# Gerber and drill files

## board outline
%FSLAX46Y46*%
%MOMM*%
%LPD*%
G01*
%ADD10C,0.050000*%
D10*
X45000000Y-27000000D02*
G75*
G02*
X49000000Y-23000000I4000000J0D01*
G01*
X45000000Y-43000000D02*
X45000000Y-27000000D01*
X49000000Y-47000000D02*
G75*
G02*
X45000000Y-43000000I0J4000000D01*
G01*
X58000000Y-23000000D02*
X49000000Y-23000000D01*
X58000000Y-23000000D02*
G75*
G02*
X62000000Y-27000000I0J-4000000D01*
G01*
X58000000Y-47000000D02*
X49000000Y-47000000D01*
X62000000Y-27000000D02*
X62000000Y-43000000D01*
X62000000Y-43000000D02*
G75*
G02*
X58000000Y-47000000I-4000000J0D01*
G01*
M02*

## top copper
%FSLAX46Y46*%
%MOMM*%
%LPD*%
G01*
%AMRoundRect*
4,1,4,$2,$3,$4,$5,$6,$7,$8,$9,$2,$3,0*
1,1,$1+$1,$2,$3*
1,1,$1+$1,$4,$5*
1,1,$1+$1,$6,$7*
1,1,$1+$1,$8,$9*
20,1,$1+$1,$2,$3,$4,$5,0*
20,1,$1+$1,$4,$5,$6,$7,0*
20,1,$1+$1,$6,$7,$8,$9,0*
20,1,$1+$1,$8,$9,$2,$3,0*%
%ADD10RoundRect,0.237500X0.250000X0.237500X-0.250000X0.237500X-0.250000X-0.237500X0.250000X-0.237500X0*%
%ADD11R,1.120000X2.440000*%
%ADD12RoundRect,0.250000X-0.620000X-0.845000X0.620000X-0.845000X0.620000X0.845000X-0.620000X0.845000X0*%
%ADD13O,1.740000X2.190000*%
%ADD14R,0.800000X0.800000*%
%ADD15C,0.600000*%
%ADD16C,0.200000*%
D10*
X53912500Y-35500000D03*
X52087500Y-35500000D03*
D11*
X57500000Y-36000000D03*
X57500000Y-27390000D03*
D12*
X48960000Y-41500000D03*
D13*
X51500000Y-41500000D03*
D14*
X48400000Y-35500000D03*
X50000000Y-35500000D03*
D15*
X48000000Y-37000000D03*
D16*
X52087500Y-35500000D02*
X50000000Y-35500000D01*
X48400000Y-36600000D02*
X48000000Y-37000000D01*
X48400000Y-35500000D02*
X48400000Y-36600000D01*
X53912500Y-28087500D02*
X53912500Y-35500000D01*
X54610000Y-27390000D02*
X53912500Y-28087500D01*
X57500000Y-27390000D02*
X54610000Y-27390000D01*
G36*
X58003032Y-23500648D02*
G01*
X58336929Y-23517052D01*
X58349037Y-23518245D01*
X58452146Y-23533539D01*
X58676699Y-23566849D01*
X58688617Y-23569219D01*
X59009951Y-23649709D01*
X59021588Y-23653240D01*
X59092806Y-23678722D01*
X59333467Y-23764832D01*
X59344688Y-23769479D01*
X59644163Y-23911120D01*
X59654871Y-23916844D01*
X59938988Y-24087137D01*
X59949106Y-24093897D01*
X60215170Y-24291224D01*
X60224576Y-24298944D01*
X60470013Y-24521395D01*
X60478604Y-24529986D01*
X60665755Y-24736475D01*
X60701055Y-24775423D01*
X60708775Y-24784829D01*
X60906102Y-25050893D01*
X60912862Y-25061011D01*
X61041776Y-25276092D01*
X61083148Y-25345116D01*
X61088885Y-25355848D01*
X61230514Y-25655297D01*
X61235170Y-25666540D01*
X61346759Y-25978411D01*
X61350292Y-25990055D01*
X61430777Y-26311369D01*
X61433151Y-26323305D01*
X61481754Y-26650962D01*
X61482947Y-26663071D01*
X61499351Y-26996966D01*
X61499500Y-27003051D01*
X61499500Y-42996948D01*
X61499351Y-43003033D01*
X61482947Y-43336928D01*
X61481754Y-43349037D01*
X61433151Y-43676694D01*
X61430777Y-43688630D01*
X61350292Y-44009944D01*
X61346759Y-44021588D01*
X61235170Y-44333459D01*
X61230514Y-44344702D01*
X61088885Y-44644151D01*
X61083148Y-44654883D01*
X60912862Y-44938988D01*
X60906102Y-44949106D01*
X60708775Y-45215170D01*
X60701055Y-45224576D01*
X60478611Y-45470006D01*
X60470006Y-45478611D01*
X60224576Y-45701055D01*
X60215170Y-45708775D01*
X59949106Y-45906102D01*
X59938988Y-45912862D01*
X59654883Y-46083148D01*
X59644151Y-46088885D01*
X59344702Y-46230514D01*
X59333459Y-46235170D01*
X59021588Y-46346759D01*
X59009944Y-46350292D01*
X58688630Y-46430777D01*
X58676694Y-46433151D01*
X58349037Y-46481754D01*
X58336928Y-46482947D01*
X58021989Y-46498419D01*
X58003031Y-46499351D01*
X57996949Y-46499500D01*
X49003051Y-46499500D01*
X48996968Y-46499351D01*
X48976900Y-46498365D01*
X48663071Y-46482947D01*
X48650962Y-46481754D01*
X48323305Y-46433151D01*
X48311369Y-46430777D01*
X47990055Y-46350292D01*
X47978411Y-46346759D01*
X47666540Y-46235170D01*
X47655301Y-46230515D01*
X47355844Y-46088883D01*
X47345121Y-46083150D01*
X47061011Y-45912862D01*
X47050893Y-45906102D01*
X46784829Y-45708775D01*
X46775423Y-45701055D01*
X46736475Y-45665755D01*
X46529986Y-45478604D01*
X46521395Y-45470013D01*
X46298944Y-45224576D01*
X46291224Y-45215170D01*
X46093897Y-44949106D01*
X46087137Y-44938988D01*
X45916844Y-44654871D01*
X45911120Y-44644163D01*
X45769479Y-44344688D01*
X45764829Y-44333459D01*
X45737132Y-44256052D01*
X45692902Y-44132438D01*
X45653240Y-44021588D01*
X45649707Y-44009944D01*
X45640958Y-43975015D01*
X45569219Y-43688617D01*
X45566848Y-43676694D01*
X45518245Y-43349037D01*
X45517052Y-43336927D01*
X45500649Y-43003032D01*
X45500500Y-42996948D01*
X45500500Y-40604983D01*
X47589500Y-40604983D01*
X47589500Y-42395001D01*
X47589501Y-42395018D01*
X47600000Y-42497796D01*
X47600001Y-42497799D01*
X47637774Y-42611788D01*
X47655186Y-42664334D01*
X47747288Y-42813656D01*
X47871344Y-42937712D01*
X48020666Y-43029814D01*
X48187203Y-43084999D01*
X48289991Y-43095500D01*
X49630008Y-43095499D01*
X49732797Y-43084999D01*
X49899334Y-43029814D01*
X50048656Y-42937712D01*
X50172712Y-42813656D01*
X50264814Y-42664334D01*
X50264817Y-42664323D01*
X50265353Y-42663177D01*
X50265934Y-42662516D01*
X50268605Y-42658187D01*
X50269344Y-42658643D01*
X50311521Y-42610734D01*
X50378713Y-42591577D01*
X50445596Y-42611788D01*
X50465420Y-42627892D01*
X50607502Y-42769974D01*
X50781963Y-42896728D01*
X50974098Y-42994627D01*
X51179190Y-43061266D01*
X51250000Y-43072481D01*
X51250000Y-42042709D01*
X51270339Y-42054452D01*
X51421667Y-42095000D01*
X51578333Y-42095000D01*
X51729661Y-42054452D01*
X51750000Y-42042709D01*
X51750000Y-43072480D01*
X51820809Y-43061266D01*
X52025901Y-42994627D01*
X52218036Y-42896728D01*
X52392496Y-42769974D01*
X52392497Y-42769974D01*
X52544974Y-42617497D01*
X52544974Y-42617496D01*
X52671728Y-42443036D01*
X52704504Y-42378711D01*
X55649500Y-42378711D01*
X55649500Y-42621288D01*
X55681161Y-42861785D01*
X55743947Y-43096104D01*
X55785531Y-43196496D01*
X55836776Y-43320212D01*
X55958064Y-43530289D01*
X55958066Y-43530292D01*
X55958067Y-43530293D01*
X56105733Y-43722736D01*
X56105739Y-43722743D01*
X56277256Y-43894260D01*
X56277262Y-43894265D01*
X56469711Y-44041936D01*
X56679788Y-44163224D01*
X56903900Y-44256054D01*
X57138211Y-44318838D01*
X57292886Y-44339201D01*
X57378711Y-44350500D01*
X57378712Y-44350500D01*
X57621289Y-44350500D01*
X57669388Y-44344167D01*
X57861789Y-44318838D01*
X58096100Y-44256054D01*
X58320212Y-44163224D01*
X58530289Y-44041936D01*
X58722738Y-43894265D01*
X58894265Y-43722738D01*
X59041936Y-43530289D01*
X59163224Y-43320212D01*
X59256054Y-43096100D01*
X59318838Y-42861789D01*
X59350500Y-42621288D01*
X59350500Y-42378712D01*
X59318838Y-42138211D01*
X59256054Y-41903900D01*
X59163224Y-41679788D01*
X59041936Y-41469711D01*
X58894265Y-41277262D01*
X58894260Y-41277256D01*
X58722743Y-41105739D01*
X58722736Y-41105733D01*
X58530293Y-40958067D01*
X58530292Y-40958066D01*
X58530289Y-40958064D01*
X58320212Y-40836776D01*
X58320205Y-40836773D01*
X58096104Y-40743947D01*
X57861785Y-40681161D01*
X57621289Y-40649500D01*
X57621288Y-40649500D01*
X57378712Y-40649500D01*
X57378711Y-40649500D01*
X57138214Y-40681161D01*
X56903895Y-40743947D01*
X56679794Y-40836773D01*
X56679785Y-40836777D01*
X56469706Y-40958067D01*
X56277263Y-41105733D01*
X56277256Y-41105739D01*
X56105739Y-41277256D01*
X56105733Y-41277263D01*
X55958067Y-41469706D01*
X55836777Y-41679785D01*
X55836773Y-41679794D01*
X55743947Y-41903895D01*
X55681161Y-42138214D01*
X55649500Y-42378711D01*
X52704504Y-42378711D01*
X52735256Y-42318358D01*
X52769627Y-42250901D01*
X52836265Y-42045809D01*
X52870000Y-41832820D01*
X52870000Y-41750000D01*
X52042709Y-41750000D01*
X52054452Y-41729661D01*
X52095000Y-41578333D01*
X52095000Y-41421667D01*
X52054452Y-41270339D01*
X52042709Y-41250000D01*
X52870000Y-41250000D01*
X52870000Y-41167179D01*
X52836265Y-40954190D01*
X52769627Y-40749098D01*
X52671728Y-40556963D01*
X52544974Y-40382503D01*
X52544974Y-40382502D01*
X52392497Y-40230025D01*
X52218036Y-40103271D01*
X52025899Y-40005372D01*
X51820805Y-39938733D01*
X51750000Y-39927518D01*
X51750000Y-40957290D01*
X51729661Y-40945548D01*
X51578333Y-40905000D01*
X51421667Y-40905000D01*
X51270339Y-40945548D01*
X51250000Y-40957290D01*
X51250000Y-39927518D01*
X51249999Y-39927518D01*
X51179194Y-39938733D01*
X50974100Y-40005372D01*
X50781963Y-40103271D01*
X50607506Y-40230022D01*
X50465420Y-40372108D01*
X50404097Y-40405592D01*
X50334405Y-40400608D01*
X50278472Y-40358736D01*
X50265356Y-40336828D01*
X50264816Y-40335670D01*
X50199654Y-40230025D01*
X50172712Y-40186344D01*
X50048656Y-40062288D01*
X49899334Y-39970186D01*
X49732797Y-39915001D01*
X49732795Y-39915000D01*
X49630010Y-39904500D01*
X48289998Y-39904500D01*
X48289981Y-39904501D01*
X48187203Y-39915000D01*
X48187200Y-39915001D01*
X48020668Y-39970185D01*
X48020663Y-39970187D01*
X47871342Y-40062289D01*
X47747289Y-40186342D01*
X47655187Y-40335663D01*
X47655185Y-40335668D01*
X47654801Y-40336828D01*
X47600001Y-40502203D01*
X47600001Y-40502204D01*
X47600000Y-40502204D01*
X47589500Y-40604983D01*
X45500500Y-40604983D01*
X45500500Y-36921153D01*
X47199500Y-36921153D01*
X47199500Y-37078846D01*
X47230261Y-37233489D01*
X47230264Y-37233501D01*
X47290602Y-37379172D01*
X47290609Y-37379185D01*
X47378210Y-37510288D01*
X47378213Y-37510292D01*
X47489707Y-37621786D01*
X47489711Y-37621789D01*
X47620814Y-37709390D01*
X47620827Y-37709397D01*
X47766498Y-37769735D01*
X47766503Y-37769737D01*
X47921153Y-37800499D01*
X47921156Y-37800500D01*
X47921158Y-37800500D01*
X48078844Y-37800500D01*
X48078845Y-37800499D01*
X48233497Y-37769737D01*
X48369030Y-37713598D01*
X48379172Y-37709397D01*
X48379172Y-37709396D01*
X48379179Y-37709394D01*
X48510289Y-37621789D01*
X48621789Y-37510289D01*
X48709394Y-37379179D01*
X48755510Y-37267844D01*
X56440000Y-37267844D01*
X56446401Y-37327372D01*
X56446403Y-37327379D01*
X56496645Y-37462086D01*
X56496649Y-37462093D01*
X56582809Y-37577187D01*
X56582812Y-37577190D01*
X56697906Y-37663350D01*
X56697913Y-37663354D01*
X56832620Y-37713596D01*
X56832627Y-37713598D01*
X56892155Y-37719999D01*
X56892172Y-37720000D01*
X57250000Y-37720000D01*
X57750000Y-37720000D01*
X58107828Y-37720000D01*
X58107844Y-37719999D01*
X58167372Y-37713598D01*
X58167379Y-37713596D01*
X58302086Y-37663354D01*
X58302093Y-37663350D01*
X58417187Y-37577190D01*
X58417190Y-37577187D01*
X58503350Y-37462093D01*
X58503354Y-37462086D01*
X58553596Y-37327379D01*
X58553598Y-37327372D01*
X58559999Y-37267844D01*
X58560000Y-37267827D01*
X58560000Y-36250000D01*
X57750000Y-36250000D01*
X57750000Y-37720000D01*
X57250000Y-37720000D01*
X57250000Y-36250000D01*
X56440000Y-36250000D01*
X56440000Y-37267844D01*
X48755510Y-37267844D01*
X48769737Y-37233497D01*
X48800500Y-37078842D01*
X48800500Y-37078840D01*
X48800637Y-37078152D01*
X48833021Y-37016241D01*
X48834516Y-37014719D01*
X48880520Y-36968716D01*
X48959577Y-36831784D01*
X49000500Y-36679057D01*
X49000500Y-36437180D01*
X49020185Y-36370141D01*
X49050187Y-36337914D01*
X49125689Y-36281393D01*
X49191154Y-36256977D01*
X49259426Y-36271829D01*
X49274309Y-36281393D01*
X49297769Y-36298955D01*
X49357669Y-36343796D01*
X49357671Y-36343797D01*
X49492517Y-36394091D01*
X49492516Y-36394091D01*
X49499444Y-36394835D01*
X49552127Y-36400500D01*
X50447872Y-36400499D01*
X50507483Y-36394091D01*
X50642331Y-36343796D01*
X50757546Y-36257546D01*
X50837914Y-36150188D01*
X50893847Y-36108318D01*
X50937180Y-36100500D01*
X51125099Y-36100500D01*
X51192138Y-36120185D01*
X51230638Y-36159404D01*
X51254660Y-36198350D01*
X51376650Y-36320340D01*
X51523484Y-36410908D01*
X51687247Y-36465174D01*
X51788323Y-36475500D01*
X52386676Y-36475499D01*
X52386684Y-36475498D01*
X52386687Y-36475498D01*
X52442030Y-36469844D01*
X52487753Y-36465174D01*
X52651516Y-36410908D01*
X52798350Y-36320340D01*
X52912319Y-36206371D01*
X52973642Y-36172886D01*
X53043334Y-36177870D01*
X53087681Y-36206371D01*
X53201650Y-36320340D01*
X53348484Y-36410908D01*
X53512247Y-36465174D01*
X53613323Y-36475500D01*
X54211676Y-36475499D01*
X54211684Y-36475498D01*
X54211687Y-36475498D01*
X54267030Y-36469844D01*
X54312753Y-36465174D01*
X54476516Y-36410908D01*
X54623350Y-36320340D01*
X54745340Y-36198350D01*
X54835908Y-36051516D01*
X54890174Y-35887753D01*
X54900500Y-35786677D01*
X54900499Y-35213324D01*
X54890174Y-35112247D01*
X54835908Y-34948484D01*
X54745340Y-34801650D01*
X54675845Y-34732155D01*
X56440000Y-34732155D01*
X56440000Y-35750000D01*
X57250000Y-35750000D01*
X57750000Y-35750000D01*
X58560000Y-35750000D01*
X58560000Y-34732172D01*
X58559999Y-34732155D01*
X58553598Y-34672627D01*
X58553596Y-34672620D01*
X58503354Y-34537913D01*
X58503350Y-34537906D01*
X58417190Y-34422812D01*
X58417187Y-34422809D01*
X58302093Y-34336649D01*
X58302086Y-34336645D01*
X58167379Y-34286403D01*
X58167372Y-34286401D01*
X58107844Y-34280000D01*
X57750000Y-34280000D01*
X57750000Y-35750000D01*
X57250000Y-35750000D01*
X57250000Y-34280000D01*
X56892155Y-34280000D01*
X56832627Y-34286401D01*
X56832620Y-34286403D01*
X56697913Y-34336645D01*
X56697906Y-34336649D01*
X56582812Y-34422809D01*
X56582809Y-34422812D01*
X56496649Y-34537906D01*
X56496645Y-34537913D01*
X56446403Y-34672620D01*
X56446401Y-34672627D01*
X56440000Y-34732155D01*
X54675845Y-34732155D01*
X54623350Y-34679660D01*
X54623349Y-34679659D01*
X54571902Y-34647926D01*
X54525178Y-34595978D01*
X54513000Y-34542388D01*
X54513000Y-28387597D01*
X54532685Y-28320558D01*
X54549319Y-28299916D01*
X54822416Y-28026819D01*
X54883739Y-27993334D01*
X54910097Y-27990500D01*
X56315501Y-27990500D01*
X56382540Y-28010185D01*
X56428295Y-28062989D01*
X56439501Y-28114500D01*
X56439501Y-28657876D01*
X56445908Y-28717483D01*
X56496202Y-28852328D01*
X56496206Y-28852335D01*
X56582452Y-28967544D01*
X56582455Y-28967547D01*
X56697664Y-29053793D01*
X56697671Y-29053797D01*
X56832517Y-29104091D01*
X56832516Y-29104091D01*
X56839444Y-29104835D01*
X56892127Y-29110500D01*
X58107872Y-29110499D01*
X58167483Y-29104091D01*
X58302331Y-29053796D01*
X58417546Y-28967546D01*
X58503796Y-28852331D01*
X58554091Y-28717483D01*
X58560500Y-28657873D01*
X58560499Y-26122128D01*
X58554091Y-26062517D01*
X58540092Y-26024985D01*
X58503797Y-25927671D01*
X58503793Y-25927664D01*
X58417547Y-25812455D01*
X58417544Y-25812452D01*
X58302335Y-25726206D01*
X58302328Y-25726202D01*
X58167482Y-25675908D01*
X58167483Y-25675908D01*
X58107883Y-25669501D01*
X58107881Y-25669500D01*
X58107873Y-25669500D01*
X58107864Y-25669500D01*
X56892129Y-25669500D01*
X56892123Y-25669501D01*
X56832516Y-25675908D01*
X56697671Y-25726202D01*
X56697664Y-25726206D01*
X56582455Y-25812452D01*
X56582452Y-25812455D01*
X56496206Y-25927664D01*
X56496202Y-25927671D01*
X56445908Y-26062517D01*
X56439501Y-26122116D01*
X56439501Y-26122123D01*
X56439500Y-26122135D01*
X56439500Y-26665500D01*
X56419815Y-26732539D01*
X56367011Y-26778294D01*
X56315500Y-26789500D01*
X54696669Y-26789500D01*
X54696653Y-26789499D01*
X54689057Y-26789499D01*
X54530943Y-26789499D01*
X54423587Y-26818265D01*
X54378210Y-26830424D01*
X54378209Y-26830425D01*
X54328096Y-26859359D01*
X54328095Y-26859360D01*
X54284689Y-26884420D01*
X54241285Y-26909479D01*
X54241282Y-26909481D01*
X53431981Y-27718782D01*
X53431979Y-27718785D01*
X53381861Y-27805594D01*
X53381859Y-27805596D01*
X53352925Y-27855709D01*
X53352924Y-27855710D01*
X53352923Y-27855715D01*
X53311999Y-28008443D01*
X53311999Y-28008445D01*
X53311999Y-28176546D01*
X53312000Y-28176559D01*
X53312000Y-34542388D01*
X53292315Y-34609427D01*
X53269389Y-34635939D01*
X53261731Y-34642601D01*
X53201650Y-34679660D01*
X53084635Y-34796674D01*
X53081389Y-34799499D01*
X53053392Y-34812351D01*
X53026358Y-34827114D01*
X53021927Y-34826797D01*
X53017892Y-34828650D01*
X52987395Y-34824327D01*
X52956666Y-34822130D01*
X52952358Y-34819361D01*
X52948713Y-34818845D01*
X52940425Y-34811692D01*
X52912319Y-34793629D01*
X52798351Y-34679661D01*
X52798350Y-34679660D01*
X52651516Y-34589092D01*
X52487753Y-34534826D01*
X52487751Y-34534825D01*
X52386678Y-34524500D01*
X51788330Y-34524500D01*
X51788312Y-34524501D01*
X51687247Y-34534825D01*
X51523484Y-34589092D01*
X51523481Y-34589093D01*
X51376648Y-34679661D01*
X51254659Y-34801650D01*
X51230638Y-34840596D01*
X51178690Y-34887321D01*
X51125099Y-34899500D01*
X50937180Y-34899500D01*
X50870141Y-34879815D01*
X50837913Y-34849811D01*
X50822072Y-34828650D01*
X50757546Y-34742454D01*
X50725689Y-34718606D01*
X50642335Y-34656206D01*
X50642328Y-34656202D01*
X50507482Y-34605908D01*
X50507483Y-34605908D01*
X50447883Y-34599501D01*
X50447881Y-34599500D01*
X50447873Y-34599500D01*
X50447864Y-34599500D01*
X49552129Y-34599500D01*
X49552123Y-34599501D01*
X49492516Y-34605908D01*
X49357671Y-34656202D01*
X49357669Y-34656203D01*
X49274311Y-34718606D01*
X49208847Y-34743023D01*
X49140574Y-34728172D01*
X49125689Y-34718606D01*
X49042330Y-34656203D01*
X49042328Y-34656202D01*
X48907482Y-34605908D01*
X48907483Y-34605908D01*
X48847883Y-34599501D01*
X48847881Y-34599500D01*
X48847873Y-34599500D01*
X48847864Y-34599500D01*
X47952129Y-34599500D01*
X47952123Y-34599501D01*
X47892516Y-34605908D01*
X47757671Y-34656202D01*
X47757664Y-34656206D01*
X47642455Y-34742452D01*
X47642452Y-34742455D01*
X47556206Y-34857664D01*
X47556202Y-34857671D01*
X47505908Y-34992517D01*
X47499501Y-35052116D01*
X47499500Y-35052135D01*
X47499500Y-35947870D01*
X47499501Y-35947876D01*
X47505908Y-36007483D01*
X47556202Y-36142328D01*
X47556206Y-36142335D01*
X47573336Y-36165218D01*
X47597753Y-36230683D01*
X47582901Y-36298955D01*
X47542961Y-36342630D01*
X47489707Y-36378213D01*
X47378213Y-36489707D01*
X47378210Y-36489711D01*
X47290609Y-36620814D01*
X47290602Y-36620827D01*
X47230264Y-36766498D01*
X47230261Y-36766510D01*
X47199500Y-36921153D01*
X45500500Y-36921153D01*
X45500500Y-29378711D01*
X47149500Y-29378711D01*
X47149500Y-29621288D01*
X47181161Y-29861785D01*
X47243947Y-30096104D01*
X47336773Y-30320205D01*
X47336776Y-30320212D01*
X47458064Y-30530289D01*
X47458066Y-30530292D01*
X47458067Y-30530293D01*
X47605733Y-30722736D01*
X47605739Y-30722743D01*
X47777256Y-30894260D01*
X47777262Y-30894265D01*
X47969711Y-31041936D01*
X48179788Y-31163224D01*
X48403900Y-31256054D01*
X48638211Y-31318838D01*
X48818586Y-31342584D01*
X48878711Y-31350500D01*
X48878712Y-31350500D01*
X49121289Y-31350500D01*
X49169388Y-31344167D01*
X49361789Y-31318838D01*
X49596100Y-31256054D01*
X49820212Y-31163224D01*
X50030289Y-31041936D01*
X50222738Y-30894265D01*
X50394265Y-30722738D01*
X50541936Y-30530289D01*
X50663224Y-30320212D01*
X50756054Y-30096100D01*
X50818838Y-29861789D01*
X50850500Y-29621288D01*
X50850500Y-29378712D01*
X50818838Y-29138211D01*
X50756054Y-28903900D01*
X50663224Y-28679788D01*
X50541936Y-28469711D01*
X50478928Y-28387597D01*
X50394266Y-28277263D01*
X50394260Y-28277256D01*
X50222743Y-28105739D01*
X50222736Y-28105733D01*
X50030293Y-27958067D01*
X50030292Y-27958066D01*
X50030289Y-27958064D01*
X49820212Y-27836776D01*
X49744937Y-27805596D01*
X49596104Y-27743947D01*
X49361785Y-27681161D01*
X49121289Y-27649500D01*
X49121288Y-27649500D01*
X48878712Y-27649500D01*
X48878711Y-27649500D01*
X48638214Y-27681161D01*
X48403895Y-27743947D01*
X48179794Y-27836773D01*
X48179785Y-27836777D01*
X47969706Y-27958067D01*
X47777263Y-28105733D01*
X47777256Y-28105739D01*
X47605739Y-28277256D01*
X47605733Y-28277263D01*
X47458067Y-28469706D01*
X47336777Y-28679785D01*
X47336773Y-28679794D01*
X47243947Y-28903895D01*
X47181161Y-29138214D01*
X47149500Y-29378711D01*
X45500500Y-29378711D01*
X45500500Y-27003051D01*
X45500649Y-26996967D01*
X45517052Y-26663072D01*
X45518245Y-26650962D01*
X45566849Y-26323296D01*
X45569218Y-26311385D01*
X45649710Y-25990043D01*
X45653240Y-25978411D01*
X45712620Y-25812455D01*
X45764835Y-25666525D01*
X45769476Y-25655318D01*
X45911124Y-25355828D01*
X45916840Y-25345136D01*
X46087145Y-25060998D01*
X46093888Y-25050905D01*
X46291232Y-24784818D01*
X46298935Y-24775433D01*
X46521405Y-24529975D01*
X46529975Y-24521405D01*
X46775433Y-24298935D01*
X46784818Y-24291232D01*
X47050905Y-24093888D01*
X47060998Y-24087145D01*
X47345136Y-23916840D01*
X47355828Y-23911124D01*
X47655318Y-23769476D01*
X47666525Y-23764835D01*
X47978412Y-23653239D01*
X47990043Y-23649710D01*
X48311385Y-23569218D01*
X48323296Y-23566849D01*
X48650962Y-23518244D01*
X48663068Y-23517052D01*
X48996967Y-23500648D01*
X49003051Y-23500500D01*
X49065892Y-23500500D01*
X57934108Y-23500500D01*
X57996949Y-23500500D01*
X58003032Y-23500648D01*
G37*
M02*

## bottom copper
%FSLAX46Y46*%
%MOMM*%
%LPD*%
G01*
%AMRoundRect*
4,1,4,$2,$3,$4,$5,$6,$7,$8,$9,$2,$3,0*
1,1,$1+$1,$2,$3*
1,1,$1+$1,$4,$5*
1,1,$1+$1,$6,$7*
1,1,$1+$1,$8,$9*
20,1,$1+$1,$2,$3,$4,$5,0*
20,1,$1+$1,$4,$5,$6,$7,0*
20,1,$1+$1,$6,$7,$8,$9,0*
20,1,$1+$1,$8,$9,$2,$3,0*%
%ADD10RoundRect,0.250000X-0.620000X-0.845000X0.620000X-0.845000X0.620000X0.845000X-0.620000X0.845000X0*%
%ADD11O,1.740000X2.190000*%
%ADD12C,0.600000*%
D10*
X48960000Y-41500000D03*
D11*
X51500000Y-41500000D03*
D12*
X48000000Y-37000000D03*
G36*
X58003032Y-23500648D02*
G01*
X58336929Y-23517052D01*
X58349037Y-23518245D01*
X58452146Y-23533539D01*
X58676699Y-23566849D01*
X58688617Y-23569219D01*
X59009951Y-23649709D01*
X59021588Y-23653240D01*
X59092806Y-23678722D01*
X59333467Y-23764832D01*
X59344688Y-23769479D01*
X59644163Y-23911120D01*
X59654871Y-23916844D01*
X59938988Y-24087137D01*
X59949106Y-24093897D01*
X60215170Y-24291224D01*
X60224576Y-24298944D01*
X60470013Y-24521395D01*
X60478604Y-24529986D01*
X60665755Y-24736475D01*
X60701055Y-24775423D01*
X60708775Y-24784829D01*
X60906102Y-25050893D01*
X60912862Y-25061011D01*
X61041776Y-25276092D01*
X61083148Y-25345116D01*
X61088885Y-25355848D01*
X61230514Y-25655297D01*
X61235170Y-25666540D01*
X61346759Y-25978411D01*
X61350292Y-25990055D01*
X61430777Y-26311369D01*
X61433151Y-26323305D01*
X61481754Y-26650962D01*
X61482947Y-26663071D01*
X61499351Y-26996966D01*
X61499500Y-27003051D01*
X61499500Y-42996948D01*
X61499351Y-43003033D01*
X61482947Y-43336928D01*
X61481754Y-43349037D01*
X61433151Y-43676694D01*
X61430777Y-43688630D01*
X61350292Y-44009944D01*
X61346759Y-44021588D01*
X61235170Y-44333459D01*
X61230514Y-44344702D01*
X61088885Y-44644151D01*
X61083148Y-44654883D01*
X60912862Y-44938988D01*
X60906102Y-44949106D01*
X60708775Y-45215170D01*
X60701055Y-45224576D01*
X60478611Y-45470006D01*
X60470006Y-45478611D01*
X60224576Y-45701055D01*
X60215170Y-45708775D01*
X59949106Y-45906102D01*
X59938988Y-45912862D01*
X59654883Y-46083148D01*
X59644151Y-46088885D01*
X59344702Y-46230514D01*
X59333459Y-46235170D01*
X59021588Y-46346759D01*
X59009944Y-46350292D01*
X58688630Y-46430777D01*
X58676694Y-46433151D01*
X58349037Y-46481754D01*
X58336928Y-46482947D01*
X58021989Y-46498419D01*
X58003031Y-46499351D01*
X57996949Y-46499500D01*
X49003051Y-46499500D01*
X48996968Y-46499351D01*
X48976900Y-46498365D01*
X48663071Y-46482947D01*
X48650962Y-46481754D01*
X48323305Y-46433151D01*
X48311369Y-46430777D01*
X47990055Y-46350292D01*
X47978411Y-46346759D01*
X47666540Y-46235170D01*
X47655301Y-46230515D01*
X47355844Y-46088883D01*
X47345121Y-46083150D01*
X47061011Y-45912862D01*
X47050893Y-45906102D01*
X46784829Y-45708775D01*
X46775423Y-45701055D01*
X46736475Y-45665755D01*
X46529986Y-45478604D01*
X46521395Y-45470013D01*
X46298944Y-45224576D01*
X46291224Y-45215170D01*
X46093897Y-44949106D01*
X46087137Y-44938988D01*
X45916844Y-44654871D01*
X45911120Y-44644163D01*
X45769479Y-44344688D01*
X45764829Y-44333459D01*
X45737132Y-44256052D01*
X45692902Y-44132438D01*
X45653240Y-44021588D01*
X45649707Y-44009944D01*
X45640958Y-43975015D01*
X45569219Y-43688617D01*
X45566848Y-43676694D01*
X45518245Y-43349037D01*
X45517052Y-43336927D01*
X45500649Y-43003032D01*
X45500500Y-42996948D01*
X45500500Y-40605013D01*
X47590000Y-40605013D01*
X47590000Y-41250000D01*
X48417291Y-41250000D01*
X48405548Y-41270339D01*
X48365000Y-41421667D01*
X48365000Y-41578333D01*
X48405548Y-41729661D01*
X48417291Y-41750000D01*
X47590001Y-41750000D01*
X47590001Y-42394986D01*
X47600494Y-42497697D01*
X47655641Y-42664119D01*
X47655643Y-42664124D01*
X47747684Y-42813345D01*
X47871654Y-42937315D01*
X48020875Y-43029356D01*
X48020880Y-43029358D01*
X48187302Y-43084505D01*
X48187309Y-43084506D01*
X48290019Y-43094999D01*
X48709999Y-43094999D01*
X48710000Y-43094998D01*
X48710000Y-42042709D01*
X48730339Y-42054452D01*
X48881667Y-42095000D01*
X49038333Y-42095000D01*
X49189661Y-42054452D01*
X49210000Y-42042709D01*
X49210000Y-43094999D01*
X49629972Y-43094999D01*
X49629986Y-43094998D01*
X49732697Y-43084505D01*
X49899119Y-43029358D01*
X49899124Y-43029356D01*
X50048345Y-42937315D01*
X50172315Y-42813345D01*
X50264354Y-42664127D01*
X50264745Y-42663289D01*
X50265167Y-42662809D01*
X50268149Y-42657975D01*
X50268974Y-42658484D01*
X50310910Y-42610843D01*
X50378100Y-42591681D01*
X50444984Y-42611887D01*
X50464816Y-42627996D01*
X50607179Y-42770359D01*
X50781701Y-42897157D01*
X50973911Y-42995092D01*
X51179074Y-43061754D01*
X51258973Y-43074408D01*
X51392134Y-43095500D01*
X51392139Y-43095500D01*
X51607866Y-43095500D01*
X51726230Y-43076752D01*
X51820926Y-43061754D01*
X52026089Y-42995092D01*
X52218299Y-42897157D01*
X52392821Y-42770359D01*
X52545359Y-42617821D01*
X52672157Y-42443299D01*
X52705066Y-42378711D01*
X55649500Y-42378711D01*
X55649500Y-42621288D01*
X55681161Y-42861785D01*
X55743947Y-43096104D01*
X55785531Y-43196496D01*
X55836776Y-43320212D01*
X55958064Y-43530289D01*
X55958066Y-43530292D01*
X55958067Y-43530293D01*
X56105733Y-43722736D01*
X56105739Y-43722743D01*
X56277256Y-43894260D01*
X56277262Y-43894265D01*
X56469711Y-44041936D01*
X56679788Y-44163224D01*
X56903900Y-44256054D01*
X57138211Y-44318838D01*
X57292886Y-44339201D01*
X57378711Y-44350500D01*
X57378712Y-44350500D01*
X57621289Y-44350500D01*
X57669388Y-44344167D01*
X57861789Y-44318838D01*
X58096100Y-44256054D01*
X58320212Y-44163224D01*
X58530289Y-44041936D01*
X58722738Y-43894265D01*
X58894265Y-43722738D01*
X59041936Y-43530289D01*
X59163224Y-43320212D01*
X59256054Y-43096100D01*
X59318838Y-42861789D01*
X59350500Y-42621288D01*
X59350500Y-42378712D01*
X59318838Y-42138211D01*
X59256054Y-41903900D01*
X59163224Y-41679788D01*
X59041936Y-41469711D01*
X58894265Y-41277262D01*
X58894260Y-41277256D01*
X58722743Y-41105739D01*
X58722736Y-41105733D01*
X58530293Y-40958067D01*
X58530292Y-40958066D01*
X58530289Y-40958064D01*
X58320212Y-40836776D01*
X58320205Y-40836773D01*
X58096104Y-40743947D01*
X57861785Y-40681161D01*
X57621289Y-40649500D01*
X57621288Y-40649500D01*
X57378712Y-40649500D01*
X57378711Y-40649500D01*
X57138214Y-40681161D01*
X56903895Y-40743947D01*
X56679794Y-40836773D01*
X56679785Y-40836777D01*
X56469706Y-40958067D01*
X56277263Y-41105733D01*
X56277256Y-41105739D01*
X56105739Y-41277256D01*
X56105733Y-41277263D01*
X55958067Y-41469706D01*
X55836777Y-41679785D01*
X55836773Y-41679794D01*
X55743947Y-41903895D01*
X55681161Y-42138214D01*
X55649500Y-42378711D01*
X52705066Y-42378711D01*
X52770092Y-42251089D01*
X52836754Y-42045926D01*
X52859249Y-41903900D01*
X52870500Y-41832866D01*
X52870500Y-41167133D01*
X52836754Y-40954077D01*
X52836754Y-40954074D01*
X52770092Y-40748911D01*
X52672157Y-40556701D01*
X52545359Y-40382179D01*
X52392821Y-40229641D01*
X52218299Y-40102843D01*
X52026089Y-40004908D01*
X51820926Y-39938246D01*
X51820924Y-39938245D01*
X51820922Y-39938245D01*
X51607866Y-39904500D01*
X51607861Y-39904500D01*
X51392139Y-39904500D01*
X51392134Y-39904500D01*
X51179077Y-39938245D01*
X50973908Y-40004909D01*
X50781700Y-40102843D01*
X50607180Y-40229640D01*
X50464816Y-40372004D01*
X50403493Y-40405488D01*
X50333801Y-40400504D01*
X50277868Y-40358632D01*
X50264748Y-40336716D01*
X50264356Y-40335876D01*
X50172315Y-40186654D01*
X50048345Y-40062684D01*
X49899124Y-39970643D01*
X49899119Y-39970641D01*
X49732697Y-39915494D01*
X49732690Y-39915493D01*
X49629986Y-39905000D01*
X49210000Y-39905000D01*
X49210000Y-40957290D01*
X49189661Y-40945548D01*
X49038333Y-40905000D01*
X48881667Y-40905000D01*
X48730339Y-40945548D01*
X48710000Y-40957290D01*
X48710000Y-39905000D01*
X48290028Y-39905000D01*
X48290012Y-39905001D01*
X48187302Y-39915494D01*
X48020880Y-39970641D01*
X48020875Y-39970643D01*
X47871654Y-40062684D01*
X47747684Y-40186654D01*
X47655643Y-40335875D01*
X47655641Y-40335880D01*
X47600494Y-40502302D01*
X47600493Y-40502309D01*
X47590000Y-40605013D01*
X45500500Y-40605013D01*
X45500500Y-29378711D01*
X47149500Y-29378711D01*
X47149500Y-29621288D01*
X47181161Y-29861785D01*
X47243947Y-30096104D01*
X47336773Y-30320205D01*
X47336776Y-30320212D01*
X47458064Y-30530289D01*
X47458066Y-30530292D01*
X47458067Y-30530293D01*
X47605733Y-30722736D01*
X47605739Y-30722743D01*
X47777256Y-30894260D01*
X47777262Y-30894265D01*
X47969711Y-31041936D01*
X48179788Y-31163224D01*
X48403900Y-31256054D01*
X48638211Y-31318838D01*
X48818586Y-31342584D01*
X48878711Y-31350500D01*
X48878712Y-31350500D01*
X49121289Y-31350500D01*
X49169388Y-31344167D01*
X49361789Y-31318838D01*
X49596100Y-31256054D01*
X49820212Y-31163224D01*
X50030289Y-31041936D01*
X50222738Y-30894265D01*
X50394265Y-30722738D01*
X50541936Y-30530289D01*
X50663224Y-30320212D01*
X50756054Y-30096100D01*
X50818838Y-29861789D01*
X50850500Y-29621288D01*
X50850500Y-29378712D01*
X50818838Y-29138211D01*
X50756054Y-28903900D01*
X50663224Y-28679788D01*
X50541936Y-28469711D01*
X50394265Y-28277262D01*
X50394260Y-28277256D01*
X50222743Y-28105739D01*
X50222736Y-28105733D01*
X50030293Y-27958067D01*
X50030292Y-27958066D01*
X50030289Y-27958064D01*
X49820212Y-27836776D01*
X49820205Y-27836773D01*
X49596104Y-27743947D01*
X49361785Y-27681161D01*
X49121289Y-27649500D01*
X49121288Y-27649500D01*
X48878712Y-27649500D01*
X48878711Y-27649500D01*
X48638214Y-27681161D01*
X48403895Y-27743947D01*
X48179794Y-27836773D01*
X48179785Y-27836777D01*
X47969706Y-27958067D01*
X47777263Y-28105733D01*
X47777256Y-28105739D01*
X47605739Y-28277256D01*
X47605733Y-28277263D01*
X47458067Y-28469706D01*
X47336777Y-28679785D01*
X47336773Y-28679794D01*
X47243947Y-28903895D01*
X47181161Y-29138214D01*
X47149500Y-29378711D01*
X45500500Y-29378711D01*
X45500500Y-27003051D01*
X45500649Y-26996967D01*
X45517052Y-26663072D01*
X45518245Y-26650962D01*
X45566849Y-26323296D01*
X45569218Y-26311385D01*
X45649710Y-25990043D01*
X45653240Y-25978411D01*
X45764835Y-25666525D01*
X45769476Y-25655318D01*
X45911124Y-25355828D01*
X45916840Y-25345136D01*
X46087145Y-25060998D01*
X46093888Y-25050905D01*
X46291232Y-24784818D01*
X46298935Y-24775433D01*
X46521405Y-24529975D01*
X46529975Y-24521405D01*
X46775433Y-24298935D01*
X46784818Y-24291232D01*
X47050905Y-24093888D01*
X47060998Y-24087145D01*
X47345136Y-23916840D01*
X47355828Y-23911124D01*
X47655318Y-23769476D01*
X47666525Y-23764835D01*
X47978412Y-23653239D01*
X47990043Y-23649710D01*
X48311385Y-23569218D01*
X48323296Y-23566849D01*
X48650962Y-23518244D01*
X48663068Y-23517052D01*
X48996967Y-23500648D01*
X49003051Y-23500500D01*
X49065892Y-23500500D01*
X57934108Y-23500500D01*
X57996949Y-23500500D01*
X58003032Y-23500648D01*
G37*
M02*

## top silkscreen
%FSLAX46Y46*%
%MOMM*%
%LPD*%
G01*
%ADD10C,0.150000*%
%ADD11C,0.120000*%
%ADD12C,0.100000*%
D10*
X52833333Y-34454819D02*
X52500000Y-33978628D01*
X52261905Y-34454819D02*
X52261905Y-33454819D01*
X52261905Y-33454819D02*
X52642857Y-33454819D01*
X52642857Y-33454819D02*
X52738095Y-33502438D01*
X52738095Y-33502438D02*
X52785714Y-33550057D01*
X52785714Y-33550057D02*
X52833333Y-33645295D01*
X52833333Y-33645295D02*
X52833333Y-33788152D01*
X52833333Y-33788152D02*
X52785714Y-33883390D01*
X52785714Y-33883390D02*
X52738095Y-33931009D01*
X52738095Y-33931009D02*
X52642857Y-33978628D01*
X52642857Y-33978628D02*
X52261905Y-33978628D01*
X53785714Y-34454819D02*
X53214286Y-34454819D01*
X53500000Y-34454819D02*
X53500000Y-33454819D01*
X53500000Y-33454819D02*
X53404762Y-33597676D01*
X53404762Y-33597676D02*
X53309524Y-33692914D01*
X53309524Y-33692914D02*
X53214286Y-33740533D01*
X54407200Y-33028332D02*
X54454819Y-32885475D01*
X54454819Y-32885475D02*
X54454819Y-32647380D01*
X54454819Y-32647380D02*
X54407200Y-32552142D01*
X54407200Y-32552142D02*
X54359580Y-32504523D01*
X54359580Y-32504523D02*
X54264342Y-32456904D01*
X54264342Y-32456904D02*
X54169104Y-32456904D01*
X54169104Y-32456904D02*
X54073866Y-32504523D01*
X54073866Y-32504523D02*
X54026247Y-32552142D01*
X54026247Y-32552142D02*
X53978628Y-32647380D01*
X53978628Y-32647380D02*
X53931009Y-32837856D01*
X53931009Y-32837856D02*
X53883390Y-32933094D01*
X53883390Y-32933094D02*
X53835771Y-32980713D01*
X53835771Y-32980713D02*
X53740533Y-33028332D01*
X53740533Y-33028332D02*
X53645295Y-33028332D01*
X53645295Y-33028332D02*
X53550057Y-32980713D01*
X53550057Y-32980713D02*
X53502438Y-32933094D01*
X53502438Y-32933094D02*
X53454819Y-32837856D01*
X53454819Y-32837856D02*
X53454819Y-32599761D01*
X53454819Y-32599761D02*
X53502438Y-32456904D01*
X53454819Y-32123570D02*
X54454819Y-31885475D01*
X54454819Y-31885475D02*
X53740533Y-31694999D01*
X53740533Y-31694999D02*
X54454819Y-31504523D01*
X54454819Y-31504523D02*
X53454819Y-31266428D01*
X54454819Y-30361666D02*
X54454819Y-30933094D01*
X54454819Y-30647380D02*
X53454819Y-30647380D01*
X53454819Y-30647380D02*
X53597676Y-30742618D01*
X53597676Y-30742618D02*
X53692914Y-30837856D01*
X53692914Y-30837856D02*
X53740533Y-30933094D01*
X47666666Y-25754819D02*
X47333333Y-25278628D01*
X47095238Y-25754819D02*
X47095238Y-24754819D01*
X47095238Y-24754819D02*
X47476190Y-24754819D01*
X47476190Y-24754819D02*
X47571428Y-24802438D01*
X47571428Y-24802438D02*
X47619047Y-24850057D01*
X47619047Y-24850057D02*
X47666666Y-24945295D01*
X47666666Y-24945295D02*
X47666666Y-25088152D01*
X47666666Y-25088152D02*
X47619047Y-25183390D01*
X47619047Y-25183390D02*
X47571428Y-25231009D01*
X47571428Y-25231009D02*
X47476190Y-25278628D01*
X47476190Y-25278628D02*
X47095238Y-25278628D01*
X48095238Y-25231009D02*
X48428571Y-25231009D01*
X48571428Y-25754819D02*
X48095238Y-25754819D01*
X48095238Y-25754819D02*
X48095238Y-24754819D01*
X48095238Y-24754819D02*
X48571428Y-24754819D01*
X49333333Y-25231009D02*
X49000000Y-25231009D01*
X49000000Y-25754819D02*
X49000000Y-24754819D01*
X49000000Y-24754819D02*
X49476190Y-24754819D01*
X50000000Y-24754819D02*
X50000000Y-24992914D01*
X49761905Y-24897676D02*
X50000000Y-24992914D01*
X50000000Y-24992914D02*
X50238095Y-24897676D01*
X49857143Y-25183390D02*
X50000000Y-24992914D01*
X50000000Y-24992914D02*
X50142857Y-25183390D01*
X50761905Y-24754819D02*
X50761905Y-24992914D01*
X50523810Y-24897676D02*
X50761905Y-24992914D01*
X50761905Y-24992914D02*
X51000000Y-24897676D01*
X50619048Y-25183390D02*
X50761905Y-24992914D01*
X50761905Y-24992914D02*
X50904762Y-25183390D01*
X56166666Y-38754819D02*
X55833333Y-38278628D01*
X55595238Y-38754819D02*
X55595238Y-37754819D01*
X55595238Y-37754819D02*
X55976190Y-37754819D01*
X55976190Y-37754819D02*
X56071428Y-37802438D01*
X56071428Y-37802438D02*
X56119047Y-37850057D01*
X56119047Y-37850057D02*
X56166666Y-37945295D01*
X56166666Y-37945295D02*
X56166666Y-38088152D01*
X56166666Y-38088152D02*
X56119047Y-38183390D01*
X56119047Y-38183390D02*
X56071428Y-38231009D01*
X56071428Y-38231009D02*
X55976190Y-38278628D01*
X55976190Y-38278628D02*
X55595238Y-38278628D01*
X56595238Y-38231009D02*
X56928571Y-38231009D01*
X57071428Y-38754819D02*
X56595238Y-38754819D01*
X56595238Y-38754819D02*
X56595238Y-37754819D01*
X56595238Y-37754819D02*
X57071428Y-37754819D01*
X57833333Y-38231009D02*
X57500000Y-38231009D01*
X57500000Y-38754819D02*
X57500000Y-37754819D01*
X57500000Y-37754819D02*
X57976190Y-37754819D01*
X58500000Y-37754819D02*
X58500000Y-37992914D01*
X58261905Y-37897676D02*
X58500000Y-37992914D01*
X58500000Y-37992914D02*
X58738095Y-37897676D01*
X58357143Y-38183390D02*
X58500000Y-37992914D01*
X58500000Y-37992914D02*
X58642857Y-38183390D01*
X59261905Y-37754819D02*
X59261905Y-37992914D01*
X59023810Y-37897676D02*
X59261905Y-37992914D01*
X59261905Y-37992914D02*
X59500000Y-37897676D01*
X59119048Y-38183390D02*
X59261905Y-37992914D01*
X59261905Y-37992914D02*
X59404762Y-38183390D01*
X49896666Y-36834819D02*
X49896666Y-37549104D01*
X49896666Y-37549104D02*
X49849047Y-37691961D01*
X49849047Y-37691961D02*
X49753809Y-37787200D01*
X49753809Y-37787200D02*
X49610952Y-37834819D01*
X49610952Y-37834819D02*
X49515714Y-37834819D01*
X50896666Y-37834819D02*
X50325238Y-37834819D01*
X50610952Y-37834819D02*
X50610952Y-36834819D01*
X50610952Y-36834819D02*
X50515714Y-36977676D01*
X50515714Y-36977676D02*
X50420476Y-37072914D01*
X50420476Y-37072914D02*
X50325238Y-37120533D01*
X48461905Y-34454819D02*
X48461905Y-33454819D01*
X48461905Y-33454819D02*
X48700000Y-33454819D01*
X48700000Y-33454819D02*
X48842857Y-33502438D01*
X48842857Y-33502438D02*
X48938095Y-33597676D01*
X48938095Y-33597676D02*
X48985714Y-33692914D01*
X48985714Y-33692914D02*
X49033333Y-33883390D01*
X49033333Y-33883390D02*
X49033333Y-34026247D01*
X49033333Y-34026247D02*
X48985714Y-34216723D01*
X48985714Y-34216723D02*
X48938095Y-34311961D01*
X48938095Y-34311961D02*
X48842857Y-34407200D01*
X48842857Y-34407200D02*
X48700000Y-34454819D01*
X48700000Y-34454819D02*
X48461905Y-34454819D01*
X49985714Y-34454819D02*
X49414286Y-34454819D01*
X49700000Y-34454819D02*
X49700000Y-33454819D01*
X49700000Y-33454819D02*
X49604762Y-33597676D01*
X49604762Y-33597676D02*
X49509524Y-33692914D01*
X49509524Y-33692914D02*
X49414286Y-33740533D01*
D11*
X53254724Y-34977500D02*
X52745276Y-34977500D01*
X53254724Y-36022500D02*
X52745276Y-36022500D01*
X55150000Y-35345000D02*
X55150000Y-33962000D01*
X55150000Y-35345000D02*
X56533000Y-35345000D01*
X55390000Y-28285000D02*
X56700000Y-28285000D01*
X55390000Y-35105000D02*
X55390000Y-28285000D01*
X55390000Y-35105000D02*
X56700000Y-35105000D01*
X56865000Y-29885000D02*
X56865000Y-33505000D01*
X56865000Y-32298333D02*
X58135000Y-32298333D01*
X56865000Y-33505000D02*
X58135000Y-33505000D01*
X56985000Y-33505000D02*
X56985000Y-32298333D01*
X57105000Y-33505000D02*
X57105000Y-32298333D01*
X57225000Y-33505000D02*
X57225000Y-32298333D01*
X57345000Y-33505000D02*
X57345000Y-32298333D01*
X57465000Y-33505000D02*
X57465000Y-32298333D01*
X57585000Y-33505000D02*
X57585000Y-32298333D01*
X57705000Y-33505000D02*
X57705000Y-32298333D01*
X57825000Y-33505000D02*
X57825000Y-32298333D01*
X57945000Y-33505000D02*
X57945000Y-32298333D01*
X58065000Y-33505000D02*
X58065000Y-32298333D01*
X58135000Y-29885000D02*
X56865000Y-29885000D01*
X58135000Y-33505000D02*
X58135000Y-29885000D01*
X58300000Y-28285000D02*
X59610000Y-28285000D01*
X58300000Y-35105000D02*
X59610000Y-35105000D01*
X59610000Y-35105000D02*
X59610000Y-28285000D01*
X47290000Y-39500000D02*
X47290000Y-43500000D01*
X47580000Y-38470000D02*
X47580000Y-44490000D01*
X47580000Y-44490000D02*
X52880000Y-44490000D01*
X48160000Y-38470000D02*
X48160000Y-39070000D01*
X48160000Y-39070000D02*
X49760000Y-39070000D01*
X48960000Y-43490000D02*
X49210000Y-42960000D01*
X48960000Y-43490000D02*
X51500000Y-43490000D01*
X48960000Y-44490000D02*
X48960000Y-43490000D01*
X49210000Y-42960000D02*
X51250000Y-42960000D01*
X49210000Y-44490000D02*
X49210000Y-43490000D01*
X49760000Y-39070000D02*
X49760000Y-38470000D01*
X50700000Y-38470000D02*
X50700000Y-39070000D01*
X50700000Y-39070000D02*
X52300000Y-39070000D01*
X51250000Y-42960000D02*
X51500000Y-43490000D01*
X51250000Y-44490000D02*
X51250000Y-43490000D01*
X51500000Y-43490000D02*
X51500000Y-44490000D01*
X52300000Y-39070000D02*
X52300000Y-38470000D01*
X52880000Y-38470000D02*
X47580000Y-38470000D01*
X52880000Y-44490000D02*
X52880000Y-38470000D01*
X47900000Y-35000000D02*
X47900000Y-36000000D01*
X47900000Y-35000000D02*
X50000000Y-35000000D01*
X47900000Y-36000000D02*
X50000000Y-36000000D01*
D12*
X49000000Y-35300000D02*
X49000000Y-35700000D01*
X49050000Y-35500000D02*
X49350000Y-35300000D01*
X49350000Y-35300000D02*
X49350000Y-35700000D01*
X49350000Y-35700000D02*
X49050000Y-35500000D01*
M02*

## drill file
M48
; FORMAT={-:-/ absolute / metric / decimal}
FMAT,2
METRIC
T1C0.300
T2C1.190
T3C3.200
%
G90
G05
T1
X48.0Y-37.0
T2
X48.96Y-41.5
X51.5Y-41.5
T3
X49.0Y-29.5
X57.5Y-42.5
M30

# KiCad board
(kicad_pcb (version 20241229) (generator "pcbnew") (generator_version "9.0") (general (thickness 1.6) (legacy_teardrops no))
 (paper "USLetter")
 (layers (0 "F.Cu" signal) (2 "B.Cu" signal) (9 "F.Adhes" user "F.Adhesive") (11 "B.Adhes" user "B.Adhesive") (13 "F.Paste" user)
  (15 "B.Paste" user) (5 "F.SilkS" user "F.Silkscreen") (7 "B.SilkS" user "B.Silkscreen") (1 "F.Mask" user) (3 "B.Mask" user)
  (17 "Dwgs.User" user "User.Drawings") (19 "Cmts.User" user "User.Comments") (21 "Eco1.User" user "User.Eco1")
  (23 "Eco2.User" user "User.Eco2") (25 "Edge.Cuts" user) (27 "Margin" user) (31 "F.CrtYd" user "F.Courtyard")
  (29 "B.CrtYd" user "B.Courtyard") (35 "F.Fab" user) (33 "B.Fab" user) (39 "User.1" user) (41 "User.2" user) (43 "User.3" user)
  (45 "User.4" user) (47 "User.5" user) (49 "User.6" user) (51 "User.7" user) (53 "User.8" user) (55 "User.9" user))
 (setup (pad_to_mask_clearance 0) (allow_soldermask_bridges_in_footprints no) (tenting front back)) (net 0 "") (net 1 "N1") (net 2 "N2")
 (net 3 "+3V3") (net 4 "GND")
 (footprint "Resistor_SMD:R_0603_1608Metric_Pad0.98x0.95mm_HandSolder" (layer "F.Cu") (at 53 35.5 180)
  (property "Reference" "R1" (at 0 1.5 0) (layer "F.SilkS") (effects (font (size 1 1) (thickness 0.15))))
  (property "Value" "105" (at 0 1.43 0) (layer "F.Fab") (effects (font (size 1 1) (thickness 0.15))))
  (fp_line (start -0.254724 0.5225) (end 0.254724 0.5225) (stroke (width 0.12) (type solid)) (layer "F.SilkS"))
  (fp_line (start -0.254724 -0.5225) (end 0.254724 -0.5225) (stroke (width 0.12) (type solid)) (layer "F.SilkS"))
  (pad "1" smd roundrect (at -0.9125 0 180) (size 0.975 0.95) (layers "F.Cu" "F.Mask" "F.Paste") (roundrect_rratio 0.25) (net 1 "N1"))
  (pad "2" smd roundrect (at 0.9125 0 180) (size 0.975 0.95) (layers "F.Cu" "F.Mask" "F.Paste") (roundrect_rratio 0.25) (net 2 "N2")))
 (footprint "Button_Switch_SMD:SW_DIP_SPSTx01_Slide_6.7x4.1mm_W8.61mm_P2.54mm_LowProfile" (layer "F.Cu") (at 57.5 31.695 90)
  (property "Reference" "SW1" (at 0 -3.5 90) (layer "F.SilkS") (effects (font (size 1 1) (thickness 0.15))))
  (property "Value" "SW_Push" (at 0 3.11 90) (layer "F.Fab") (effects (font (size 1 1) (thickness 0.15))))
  (fp_line (start -3.65 -2.35) (end -2.267 -2.35) (stroke (width 0.12) (type solid)) (layer "F.SilkS"))
  (fp_line (start -3.65 -2.35) (end -3.65 -0.967) (stroke (width 0.12) (type solid)) (layer "F.SilkS"))
  (fp_line (start 3.41 -2.11) (end 3.41 -0.8) (stroke (width 0.12) (type solid)) (layer "F.SilkS"))
  (fp_line (start -3.41 -2.11) (end 3.41 -2.11) (stroke (width 0.12) (type solid)) (layer "F.SilkS"))
  (fp_line (start -3.41 -2.11) (end -3.41 -0.8) (stroke (width 0.12) (type solid)) (layer "F.SilkS"))
  (fp_line (start 1.81 -0.635) (end -1.81 -0.635) (stroke (width 0.12) (type solid)) (layer "F.SilkS"))
  (fp_line (start -0.603333 -0.635) (end -0.603333 0.635) (stroke (width 0.12) (type solid)) (layer "F.SilkS"))
  (fp_line (start -1.81 -0.635) (end -1.81 0.635) (stroke (width 0.12) (type solid)) (layer "F.SilkS"))
  (fp_line (start -1.81 -0.515) (end -0.603333 -0.515) (stroke (width 0.12) (type solid)) (layer "F.SilkS"))
  (fp_line (start -1.81 -0.395) (end -0.603333 -0.395) (stroke (width 0.12) (type solid)) (layer "F.SilkS"))
  (fp_line (start -1.81 -0.275) (end -0.603333 -0.275) (stroke (width 0.12) (type solid)) (layer "F.SilkS"))
  (fp_line (start -1.81 -0.155) (end -0.603333 -0.155) (stroke (width 0.12) (type solid)) (layer "F.SilkS"))
  (fp_line (start -1.81 -0.035) (end -0.603333 -0.035) (stroke (width 0.12) (type solid)) (layer "F.SilkS"))
  (fp_line (start -1.81 0.085) (end -0.603333 0.085) (stroke (width 0.12) (type solid)) (layer "F.SilkS"))
  (fp_line (start -1.81 0.205) (end -0.603333 0.205) (stroke (width 0.12) (type solid)) (layer "F.SilkS"))
  (fp_line (start -1.81 0.325) (end -0.603333 0.325) (stroke (width 0.12) (type solid)) (layer "F.SilkS"))
  (fp_line (start -1.81 0.445) (end -0.603333 0.445) (stroke (width 0.12) (type solid)) (layer "F.SilkS"))
  (fp_line (start -1.81 0.565) (end -0.603333 0.565) (stroke (width 0.12) (type solid)) (layer "F.SilkS"))
  (fp_line (start 1.81 0.635) (end 1.81 -0.635) (stroke (width 0.12) (type solid)) (layer "F.SilkS"))
  (fp_line (start -1.81 0.635) (end 1.81 0.635) (stroke (width 0.12) (type solid)) (layer "F.SilkS"))
  (fp_line (start 3.41 0.8) (end 3.41 2.11) (stroke (width 0.12) (type solid)) (layer "F.SilkS"))
  (fp_line (start -3.41 0.8) (end -3.41 2.11) (stroke (width 0.12) (type solid)) (layer "F.SilkS"))
  (fp_line (start -3.41 2.11) (end 3.41 2.11) (stroke (width 0.12) (type solid)) (layer "F.SilkS"))
  (pad "1" smd rect (at -4.305 0 90) (size 2.44 1.12) (layers "F.Cu" "F.Mask" "F.Paste") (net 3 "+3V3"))
  (pad "2" smd rect (at 4.305 0 90) (size 2.44 1.12) (layers "F.Cu" "F.Mask" "F.Paste") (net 1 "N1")))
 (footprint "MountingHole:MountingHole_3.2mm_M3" (layer "F.Cu") (at 49 29.5)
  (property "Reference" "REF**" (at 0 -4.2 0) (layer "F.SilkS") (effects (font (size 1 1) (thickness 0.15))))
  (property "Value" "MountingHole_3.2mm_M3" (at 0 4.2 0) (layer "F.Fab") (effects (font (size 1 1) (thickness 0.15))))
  (pad "" np_thru_hole circle (at 0 0) (size 3.2 3.2) (drill 3.2) (layers "*.Cu" "*.Mask")))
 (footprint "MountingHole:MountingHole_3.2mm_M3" (layer "F.Cu") (at 57.5 42.5)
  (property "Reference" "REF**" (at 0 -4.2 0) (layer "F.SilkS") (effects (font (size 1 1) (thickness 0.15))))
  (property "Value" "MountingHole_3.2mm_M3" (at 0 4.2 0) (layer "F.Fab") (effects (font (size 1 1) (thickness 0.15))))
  (pad "" np_thru_hole circle (at 0 0) (size 3.2 3.2) (drill 3.2) (layers "*.Cu" "*.Mask")))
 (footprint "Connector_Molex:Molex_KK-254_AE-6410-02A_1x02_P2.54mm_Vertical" (layer "F.Cu") (at 48.96 41.5)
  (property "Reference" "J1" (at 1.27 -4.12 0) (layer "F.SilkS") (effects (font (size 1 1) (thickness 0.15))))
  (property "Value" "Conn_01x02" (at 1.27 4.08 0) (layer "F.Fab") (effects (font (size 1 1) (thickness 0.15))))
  (fp_line (start -1.67 -2) (end -1.67 2) (stroke (width 0.12) (type solid)) (layer "F.SilkS"))
  (fp_line (start -1.38 -3.03) (end -1.38 2.99) (stroke (width 0.12) (type solid)) (layer "F.SilkS"))
  (fp_line (start -1.38 2.99) (end 3.92 2.99) (stroke (width 0.12) (type solid)) (layer "F.SilkS"))
  (fp_line (start -0.8 -3.03) (end -0.8 -2.43) (stroke (width 0.12) (type solid)) (layer "F.SilkS"))
  (fp_line (start -0.8 -2.43) (end 0.8 -2.43) (stroke (width 0.12) (type solid)) (layer "F.SilkS"))
  (fp_line (start 0 1.99) (end 0.25 1.46) (stroke (width 0.12) (type solid)) (layer "F.SilkS"))
  (fp_line (start 0 1.99) (end 2.54 1.99) (stroke (width 0.12) (type solid)) (layer "F.SilkS"))
  (fp_line (start 0 2.99) (end 0 1.99) (stroke (width 0.12) (type solid)) (layer "F.SilkS"))
  (fp_line (start 0.25 1.46) (end 2.29 1.46) (stroke (width 0.12) (type solid)) (layer "F.SilkS"))
  (fp_line (start 0.25 2.99) (end 0.25 1.99) (stroke (width 0.12) (type solid)) (layer "F.SilkS"))
  (fp_line (start 0.8 -2.43) (end 0.8 -3.03) (stroke (width 0.12) (type solid)) (layer "F.SilkS"))
  (fp_line (start 1.74 -3.03) (end 1.74 -2.43) (stroke (width 0.12) (type solid)) (layer "F.SilkS"))
  (fp_line (start 1.74 -2.43) (end 3.34 -2.43) (stroke (width 0.12) (type solid)) (layer "F.SilkS"))
  (fp_line (start 2.29 1.46) (end 2.54 1.99) (stroke (width 0.12) (type solid)) (layer "F.SilkS"))
  (fp_line (start 2.29 2.99) (end 2.29 1.99) (stroke (width 0.12) (type solid)) (layer "F.SilkS"))
  (fp_line (start 2.54 1.99) (end 2.54 2.99) (stroke (width 0.12) (type solid)) (layer "F.SilkS"))
  (fp_line (start 3.34 -2.43) (end 3.34 -3.03) (stroke (width 0.12) (type solid)) (layer "F.SilkS"))
  (fp_line (start 3.92 -3.03) (end -1.38 -3.03) (stroke (width 0.12) (type solid)) (layer "F.SilkS"))
  (fp_line (start 3.92 2.99) (end 3.92 -3.03) (stroke (width 0.12) (type solid)) (layer "F.SilkS"))
  (pad "1" thru_hole roundrect (at 0 0) (size 1.74 2.19) (drill 1.19) (layers "*.Cu" "*.Mask") (remove_unused_layers no)
   (roundrect_rratio 0.143678) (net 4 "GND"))
  (pad "2" thru_hole oval (at 2.54 0) (size 1.74 2.19) (drill 1.19) (layers "*.Cu" "*.Mask") (remove_unused_layers no) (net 3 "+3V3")))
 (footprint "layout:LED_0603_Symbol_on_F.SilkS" (layer "F.Cu") (at 49.2 35.5)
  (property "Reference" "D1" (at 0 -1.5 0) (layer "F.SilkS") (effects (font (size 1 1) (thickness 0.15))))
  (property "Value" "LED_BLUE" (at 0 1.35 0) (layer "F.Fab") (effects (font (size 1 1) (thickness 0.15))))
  (fp_line (start -1.3 -0.5) (end -1.3 0.5) (stroke (width 0.12) (type solid)) (layer "F.SilkS"))
  (fp_line (start -1.3 -0.5) (end 0.8 -0.5) (stroke (width 0.12) (type solid)) (layer "F.SilkS"))
  (fp_line (start -1.3 0.5) (end 0.8 0.5) (stroke (width 0.12) (type solid)) (layer "F.SilkS"))
  (fp_line (start -0.2 -0.2) (end -0.2 0.2) (stroke (width 0.1) (type solid)) (layer "F.SilkS"))
  (fp_line (start -0.15 0) (end 0.15 -0.2) (stroke (width 0.1) (type solid)) (layer "F.SilkS"))
  (fp_line (start 0.15 -0.2) (end 0.15 0.2) (stroke (width 0.1) (type solid)) (layer "F.SilkS"))
  (fp_line (start 0.15 0.2) (end -0.15 0) (stroke (width 0.1) (type solid)) (layer "F.SilkS"))
  (pad "1" smd rect (at -0.8 0 180) (size 0.8 0.8) (layers "F.Cu" "F.Mask" "F.Paste") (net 4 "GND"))
  (pad "2" smd rect (at 0.8 0 180) (size 0.8 0.8) (layers "F.Cu" "F.Mask" "F.Paste") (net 2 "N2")))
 (gr_arc (start 45 27) (mid 46.171573 24.171573) (end 49 23) (stroke (width 0.05) (type default)) (layer "Edge.Cuts"))
 (gr_line (start 45 43) (end 45 27) (stroke (width 0.05) (type default)) (layer "Edge.Cuts"))
 (gr_arc (start 49 47) (mid 46.171573 45.828427) (end 45 43) (stroke (width 0.05) (type default)) (layer "Edge.Cuts"))
 (gr_line (start 58 23) (end 49 23) (stroke (width 0.05) (type default)) (layer "Edge.Cuts"))
 (gr_arc (start 58 23) (mid 60.828427 24.171573) (end 62 27) (stroke (width 0.05) (type default)) (layer "Edge.Cuts"))
 (gr_line (start 58 47) (end 49 47) (stroke (width 0.05) (type default)) (layer "Edge.Cuts"))
 (gr_line (start 62 27) (end 62 43) (stroke (width 0.05) (type default)) (layer "Edge.Cuts"))
 (gr_arc (start 62 43) (mid 60.828427 45.828427) (end 58 47) (stroke (width 0.05) (type default)) (layer "Edge.Cuts"))
 (segment (start 52.0875 35.5) (end 50 35.5) (width 0.2) (layer "F.Cu") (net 2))
 (segment (start 48.4 36.6) (end 48 37) (width 0.2) (layer "F.Cu") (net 4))
 (segment (start 48.4 35.5) (end 48.4 36.6) (width 0.2) (layer "F.Cu") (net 4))
 (via (at 48 37) (size 0.6) (drill 0.3) (layers "F.Cu" "B.Cu") (free yes) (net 4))
 (segment (start 53.9125 28.0875) (end 53.9125 35.5) (width 0.2) (layer "F.Cu") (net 1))
 (segment (start 54.61 27.39) (end 53.9125 28.0875) (width 0.2) (layer "F.Cu") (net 1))
 (segment (start 57.5 27.39) (end 54.61 27.39) (width 0.2) (layer "F.Cu") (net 1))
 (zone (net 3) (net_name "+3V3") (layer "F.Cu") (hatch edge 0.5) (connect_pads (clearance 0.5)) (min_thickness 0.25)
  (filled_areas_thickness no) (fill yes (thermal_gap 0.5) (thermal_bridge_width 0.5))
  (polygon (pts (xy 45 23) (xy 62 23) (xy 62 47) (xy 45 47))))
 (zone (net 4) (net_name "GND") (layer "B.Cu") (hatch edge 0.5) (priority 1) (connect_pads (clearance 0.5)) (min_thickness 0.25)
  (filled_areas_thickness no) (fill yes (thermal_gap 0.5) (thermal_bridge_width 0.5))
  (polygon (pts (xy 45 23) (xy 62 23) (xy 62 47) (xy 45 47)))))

